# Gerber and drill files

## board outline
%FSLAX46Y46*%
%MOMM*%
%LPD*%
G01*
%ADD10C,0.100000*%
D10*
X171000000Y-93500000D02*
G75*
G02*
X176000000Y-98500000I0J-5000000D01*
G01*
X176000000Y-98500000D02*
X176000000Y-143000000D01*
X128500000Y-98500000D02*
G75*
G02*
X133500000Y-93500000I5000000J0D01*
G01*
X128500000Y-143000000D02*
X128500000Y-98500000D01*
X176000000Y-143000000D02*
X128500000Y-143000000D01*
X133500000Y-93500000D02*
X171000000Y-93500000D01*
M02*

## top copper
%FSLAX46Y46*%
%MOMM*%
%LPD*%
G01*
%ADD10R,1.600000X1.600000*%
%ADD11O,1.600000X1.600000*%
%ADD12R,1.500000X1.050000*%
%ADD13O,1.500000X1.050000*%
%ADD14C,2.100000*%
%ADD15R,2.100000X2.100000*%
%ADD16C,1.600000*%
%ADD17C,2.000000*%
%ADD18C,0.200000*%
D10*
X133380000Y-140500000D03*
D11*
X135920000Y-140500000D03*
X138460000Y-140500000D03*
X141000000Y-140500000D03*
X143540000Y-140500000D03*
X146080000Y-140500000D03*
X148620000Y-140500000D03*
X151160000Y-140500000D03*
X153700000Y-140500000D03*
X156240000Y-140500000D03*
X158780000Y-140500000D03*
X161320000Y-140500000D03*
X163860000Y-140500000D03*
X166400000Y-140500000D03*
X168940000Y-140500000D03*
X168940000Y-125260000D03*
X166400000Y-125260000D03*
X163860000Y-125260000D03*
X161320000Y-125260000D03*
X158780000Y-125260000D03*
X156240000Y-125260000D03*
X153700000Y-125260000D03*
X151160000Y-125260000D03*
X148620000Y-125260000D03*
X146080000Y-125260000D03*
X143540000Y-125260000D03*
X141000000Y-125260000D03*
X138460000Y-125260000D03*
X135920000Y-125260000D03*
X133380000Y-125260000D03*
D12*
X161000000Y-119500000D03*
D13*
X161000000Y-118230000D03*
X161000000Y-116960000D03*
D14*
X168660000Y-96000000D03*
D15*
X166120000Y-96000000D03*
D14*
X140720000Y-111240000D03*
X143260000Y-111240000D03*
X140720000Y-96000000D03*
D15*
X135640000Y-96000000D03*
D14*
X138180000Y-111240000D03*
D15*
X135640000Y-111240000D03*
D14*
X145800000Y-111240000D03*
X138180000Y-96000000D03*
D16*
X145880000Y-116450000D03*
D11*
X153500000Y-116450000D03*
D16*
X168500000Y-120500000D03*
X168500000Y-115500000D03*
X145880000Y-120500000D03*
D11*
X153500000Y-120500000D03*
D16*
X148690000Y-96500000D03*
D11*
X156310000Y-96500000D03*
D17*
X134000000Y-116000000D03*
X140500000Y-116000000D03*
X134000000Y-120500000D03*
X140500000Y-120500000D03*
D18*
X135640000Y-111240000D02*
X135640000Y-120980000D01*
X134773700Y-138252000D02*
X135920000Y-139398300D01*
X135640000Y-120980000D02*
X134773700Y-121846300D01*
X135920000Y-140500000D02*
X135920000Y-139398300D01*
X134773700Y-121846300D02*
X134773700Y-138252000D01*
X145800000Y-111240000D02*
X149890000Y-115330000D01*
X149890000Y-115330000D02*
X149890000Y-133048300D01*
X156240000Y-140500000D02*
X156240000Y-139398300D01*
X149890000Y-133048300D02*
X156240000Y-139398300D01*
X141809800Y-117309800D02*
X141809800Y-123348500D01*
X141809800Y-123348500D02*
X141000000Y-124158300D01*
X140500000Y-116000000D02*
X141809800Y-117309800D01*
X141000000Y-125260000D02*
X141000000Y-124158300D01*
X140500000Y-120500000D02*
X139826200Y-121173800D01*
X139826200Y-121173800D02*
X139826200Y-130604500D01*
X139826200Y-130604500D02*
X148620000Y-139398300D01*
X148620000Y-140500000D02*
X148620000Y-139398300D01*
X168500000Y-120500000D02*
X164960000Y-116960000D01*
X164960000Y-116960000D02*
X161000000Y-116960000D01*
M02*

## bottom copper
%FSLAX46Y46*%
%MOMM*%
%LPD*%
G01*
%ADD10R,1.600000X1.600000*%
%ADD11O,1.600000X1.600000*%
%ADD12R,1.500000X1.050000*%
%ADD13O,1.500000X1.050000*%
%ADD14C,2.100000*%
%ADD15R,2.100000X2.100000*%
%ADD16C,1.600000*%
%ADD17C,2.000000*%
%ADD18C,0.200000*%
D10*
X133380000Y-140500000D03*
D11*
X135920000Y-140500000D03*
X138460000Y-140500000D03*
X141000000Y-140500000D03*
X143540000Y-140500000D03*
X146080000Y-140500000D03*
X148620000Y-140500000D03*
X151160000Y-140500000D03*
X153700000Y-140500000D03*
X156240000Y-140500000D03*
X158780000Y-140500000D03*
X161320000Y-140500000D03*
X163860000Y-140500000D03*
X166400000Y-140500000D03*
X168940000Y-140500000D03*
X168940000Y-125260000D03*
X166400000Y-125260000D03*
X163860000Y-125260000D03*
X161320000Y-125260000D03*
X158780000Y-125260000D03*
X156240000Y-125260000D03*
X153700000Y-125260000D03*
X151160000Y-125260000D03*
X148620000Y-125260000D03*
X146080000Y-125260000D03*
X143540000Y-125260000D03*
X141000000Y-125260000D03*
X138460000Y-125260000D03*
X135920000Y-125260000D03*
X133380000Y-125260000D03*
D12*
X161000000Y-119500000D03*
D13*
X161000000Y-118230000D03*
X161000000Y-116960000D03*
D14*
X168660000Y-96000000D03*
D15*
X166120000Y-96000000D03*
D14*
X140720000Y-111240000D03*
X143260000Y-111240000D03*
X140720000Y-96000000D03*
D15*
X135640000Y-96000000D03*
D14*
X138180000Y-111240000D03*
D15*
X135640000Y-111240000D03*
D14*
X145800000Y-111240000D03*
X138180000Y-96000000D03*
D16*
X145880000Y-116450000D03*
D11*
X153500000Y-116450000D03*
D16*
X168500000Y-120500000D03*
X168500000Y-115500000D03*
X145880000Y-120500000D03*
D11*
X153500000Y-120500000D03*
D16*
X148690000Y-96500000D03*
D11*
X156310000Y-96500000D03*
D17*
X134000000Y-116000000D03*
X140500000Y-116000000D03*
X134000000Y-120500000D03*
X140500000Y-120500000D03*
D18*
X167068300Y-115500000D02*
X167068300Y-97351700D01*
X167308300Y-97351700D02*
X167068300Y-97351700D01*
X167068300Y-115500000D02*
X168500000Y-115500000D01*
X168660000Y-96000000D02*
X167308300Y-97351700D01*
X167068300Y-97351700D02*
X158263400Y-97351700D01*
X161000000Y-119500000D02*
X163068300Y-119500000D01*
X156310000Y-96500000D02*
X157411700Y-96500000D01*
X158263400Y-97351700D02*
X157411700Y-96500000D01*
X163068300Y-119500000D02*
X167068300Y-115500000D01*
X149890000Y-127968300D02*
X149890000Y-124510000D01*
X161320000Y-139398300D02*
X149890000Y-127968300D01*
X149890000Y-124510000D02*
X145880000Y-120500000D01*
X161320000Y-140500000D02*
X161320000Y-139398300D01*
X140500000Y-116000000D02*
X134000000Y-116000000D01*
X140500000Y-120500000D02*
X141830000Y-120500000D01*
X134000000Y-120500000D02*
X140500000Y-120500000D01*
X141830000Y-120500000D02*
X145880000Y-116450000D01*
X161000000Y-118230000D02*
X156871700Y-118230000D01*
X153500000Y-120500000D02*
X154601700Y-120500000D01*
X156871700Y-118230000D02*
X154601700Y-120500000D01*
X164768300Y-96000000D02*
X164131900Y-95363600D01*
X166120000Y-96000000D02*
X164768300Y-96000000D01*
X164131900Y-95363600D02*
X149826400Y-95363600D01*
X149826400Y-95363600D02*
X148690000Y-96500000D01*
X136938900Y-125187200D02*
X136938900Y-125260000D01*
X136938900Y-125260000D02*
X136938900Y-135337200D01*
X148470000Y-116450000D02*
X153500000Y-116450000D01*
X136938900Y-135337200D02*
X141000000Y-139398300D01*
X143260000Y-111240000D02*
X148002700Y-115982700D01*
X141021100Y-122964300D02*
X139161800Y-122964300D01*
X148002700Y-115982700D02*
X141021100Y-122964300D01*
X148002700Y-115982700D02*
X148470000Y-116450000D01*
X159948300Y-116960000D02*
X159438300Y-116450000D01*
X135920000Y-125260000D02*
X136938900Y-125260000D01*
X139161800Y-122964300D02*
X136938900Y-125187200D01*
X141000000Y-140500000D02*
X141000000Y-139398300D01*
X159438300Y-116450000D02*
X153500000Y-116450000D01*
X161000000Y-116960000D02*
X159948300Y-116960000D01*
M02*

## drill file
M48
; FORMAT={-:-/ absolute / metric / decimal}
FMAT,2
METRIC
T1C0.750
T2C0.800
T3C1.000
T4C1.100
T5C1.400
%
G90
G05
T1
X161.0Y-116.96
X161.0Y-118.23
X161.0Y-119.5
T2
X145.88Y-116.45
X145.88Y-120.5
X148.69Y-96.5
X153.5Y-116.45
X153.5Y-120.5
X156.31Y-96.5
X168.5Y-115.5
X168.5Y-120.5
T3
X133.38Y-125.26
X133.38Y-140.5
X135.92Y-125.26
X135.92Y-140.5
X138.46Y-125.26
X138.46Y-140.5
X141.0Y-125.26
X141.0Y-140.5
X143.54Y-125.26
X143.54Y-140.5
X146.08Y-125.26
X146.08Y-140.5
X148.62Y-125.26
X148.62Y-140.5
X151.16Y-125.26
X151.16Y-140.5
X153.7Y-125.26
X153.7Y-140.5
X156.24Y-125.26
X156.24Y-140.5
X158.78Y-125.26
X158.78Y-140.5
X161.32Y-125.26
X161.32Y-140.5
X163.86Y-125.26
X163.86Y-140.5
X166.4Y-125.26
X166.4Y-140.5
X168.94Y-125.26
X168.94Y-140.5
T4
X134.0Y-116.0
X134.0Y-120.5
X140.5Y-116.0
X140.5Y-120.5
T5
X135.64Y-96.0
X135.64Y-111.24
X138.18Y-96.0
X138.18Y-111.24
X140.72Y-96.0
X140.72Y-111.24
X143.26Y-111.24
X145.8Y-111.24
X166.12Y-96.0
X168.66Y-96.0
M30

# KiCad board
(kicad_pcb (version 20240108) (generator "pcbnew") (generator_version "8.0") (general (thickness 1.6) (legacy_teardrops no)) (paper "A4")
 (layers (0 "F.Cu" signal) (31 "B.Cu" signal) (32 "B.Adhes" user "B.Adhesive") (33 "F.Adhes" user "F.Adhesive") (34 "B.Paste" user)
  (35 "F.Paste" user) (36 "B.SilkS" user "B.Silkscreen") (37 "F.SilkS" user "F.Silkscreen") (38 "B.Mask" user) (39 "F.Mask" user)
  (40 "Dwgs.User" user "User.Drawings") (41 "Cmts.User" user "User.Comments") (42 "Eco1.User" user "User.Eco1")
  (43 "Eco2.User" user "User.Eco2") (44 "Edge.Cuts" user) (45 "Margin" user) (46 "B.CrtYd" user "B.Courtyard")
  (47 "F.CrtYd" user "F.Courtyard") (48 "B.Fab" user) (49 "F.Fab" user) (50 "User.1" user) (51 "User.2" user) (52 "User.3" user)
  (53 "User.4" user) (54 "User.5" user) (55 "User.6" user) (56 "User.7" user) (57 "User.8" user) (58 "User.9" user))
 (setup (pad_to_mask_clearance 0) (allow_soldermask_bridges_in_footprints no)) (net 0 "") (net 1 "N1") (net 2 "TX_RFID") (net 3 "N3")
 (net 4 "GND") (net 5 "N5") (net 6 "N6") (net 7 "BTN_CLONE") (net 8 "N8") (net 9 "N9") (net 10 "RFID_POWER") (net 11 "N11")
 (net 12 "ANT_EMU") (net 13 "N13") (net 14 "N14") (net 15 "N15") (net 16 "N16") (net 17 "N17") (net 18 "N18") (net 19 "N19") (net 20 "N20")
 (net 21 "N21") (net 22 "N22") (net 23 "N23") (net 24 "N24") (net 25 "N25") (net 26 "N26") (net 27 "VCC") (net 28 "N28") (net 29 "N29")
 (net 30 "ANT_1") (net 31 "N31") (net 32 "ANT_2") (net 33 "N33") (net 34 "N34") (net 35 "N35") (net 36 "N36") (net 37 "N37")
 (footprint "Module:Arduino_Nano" (layer "F.Cu") (at 133.38 140.5 90)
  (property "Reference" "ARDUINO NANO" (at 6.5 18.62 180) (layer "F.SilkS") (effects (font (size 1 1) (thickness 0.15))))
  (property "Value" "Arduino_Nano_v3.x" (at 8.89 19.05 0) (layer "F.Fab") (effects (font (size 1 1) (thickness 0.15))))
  (pad "1" thru_hole rect (at 0 0 90) (size 1.6 1.6) (drill 1) (layers "*.Cu" "*.Mask") (remove_unused_layers no) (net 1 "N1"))
  (pad "2" thru_hole oval (at 0 2.54 90) (size 1.6 1.6) (drill 1) (layers "*.Cu" "*.Mask") (remove_unused_layers no) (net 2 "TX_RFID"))
  (pad "3" thru_hole oval (at 0 5.08 90) (size 1.6 1.6) (drill 1) (layers "*.Cu" "*.Mask") (remove_unused_layers no) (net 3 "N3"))
  (pad "4" thru_hole oval (at 0 7.62 90) (size 1.6 1.6) (drill 1) (layers "*.Cu" "*.Mask") (remove_unused_layers no) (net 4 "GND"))
  (pad "5" thru_hole oval (at 0 10.16 90) (size 1.6 1.6) (drill 1) (layers "*.Cu" "*.Mask") (remove_unused_layers no) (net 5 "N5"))
  (pad "6" thru_hole oval (at 0 12.7 90) (size 1.6 1.6) (drill 1) (layers "*.Cu" "*.Mask") (remove_unused_layers no) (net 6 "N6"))
  (pad "7" thru_hole oval (at 0 15.24 90) (size 1.6 1.6) (drill 1) (layers "*.Cu" "*.Mask") (remove_unused_layers no) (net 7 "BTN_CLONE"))
  (pad "8" thru_hole oval (at 0 17.78 90) (size 1.6 1.6) (drill 1) (layers "*.Cu" "*.Mask") (remove_unused_layers no) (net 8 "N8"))
  (pad "9" thru_hole oval (at 0 20.32 90) (size 1.6 1.6) (drill 1) (layers "*.Cu" "*.Mask") (remove_unused_layers no) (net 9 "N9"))
  (pad "10" thru_hole oval (at 0 22.86 90) (size 1.6 1.6) (drill 1) (layers "*.Cu" "*.Mask") (remove_unused_layers no) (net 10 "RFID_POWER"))
  (pad "11" thru_hole oval (at 0 25.4 90) (size 1.6 1.6) (drill 1) (layers "*.Cu" "*.Mask") (remove_unused_layers no) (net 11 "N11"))
  (pad "12" thru_hole oval (at 0 27.94 90) (size 1.6 1.6) (drill 1) (layers "*.Cu" "*.Mask") (remove_unused_layers no) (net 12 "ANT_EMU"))
  (pad "13" thru_hole oval (at 0 30.48 90) (size 1.6 1.6) (drill 1) (layers "*.Cu" "*.Mask") (remove_unused_layers no) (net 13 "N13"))
  (pad "14" thru_hole oval (at 0 33.02 90) (size 1.6 1.6) (drill 1) (layers "*.Cu" "*.Mask") (remove_unused_layers no) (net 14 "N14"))
  (pad "15" thru_hole oval (at 0 35.56 90) (size 1.6 1.6) (drill 1) (layers "*.Cu" "*.Mask") (remove_unused_layers no) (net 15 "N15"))
  (pad "16" thru_hole oval (at 15.24 35.56 90) (size 1.6 1.6) (drill 1) (layers "*.Cu" "*.Mask") (remove_unused_layers no) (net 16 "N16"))
  (pad "17" thru_hole oval (at 15.24 33.02 90) (size 1.6 1.6) (drill 1) (layers "*.Cu" "*.Mask") (remove_unused_layers no) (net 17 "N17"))
  (pad "18" thru_hole oval (at 15.24 30.48 90) (size 1.6 1.6) (drill 1) (layers "*.Cu" "*.Mask") (remove_unused_layers no) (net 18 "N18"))
  (pad "19" thru_hole oval (at 15.24 27.94 90) (size 1.6 1.6) (drill 1) (layers "*.Cu" "*.Mask") (remove_unused_layers no) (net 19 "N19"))
  (pad "20" thru_hole oval (at 15.24 25.4 90) (size 1.6 1.6) (drill 1) (layers "*.Cu" "*.Mask") (remove_unused_layers no) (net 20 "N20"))
  (pad "21" thru_hole oval (at 15.24 22.86 90) (size 1.6 1.6) (drill 1) (layers "*.Cu" "*.Mask") (remove_unused_layers no) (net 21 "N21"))
  (pad "22" thru_hole oval (at 15.24 20.32 90) (size 1.6 1.6) (drill 1) (layers "*.Cu" "*.Mask") (remove_unused_layers no) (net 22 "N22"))
  (pad "23" thru_hole oval (at 15.24 17.78 90) (size 1.6 1.6) (drill 1) (layers "*.Cu" "*.Mask") (remove_unused_layers no) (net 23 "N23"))
  (pad "24" thru_hole oval (at 15.24 15.24 90) (size 1.6 1.6) (drill 1) (layers "*.Cu" "*.Mask") (remove_unused_layers no) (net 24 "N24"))
  (pad "25" thru_hole oval (at 15.24 12.7 90) (size 1.6 1.6) (drill 1) (layers "*.Cu" "*.Mask") (remove_unused_layers no) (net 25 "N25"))
  (pad "26" thru_hole oval (at 15.24 10.16 90) (size 1.6 1.6) (drill 1) (layers "*.Cu" "*.Mask") (remove_unused_layers no) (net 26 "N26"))
  (pad "27" thru_hole oval (at 15.24 7.62 90) (size 1.6 1.6) (drill 1) (layers "*.Cu" "*.Mask") (remove_unused_layers no) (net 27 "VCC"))
  (pad "28" thru_hole oval (at 15.24 5.08 90) (size 1.6 1.6) (drill 1) (layers "*.Cu" "*.Mask") (remove_unused_layers no) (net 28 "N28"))
  (pad "29" thru_hole oval (at 15.24 2.54 90) (size 1.6 1.6) (drill 1) (layers "*.Cu" "*.Mask") (remove_unused_layers no) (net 4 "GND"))
  (pad "30" thru_hole oval (at 15.24 0 90) (size 1.6 1.6) (drill 1) (layers "*.Cu" "*.Mask") (remove_unused_layers no) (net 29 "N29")))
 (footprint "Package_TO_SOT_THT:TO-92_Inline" (layer "F.Cu") (at 161 119.5 90)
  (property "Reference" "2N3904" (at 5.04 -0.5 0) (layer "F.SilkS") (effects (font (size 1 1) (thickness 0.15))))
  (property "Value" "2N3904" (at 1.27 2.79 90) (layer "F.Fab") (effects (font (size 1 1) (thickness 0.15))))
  (pad "1" thru_hole rect (at 0 0 90) (size 1.05 1.5) (drill 0.75) (layers "*.Cu" "*.Mask") (remove_unused_layers no) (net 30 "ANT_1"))
  (pad "2" thru_hole oval (at 1.27 0 90) (size 1.05 1.5) (drill 0.75) (layers "*.Cu" "*.Mask") (remove_unused_layers no) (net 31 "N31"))
  (pad "3" thru_hole oval (at 2.54 0 90) (size 1.05 1.5) (drill 0.75) (layers "*.Cu" "*.Mask") (remove_unused_layers no) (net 4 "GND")))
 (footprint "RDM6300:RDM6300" (layer "F.Cu") (at 152.15 103.62 180)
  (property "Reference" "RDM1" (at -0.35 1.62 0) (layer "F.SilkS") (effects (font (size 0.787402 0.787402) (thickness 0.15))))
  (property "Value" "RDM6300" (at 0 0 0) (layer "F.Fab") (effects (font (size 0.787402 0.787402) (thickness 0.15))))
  (pad "ANT1" thru_hole circle (at -16.51 7.62 180) (size 2.1 2.1) (drill 1.4) (layers "*.Cu" "*.Mask") (remove_unused_layers no)
   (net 30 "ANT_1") (solder_mask_margin 0.102))
  (pad "ANT2" thru_hole rect (at -13.97 7.62 180) (size 2.1 2.1) (drill 1.4) (layers "*.Cu" "*.Mask") (remove_unused_layers no)
   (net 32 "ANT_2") (solder_mask_margin 0.102))
  (pad "D0" thru_hole circle (at 11.43 -7.62 180) (size 2.1 2.1) (drill 1.4) (layers "*.Cu" "*.Mask") (remove_unused_layers no)
   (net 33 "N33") (solder_mask_margin 0.102))
  (pad "GND" thru_hole circle (at 8.89 -7.62 180) (size 2.1 2.1) (drill 1.4) (layers "*.Cu" "*.Mask") (remove_unused_layers no)
   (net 4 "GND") (solder_mask_margin 0.102))
  (pad "GND1" thru_hole circle (at 11.43 7.62 180) (size 2.1 2.1) (drill 1.4) (layers "*.Cu" "*.Mask") (remove_unused_layers no)
   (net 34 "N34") (solder_mask_margin 0.102))
  (pad "LED" thru_hole rect (at 16.51 7.62 180) (size 2.1 2.1) (drill 1.4) (layers "*.Cu" "*.Mask") (remove_unused_layers no) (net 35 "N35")
   (solder_mask_margin 0.102))
  (pad "RX" thru_hole circle (at 13.97 -7.62 180) (size 2.1 2.1) (drill 1.4) (layers "*.Cu" "*.Mask") (remove_unused_layers no)
   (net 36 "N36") (solder_mask_margin 0.102))
  (pad "TX" thru_hole rect (at 16.51 -7.62 180) (size 2.1 2.1) (drill 1.4) (layers "*.Cu" "*.Mask") (remove_unused_layers no)
   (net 2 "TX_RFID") (solder_mask_margin 0.102))
  (pad "VCC" thru_hole circle (at 6.35 -7.62 180) (size 2.1 2.1) (drill 1.4) (layers "*.Cu" "*.Mask") (remove_unused_layers no)
   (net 10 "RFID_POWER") (solder_mask_margin 0.102))
  (pad "VCC1" thru_hole circle (at 13.97 7.62 180) (size 2.1 2.1) (drill 1.4) (layers "*.Cu" "*.Mask") (remove_unused_layers no)
   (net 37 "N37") (solder_mask_margin 0.102)))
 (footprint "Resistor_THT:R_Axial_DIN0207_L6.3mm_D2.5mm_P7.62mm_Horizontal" (layer "F.Cu") (at 145.88 116.45)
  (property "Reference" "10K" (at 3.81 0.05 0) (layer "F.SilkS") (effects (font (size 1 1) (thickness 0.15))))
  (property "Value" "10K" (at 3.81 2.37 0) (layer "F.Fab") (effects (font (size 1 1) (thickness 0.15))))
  (pad "1" thru_hole circle (at 0 0) (size 1.6 1.6) (drill 0.8) (layers "*.Cu" "*.Mask") (remove_unused_layers no) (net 7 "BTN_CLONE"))
  (pad "2" thru_hole oval (at 7.62 0) (size 1.6 1.6) (drill 0.8) (layers "*.Cu" "*.Mask") (remove_unused_layers no) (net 4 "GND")))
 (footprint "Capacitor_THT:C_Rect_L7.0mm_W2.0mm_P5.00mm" (layer "F.Cu") (at 168.5 120.5 90)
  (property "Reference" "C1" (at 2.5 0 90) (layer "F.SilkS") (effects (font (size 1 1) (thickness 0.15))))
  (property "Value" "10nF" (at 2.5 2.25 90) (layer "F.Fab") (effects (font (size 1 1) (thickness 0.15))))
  (pad "1" thru_hole circle (at 0 0 90) (size 1.6 1.6) (drill 0.8) (layers "*.Cu" "*.Mask") (remove_unused_layers no) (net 4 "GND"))
  (pad "2" thru_hole circle (at 5 0 90) (size 1.6 1.6) (drill 0.8) (layers "*.Cu" "*.Mask") (remove_unused_layers no) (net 30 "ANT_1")))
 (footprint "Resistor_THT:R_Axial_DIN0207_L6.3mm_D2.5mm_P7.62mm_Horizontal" (layer "F.Cu") (at 145.88 120.5)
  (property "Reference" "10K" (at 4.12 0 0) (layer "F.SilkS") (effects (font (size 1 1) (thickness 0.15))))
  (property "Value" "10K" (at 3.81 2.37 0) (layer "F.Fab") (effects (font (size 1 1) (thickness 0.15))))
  (pad "1" thru_hole circle (at 0 0) (size 1.6 1.6) (drill 0.8) (layers "*.Cu" "*.Mask") (remove_unused_layers no) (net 12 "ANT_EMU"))
  (pad "2" thru_hole oval (at 7.62 0) (size 1.6 1.6) (drill 0.8) (layers "*.Cu" "*.Mask") (remove_unused_layers no) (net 31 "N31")))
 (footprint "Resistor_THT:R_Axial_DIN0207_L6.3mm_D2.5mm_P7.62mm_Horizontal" (layer "F.Cu") (at 148.69 96.5)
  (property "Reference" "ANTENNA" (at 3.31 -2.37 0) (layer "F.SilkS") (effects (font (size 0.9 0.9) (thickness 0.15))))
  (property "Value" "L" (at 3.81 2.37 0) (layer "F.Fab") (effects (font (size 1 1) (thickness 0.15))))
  (pad "1" thru_hole circle (at 0 0) (size 1.6 1.6) (drill 0.8) (layers "*.Cu" "*.Mask") (remove_unused_layers no) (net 32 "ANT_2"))
  (pad "2" thru_hole oval (at 7.62 0) (size 1.6 1.6) (drill 0.8) (layers "*.Cu" "*.Mask") (remove_unused_layers no) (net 30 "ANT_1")))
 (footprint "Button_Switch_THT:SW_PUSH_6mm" (layer "F.Cu") (at 134 116)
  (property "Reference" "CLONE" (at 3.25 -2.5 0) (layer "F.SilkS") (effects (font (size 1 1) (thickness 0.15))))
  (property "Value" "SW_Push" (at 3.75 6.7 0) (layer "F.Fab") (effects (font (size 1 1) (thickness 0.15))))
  (pad "1" thru_hole circle (at 0 0 90) (size 2 2) (drill 1.1) (layers "*.Cu" "*.Mask") (remove_unused_layers no) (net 27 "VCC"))
  (pad "1" thru_hole circle (at 6.5 0 90) (size 2 2) (drill 1.1) (layers "*.Cu" "*.Mask") (remove_unused_layers no) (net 27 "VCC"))
  (pad "2" thru_hole circle (at 0 4.5 90) (size 2 2) (drill 1.1) (layers "*.Cu" "*.Mask") (remove_unused_layers no) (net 7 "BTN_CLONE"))
  (pad "2" thru_hole circle (at 6.5 4.5 90) (size 2 2) (drill 1.1) (layers "*.Cu" "*.Mask") (remove_unused_layers no) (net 7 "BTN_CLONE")))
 (gr_arc (start 171 93.5) (mid 174.535534 94.964466) (end 176 98.5) (stroke (width 0.1) (type default)) (layer "Edge.Cuts"))
 (gr_line (start 176 98.5) (end 176 143) (stroke (width 0.1) (type default)) (layer "Edge.Cuts"))
 (gr_arc (start 128.5 98.5) (mid 129.964466 94.964466) (end 133.5 93.5) (stroke (width 0.1) (type default)) (layer "Edge.Cuts"))
 (gr_line (start 128.5 143) (end 128.5 98.5) (stroke (width 0.1) (type default)) (layer "Edge.Cuts"))
 (gr_line (start 176 143) (end 128.5 143) (stroke (width 0.1) (type default)) (layer "Edge.Cuts"))
 (gr_line (start 133.5 93.5) (end 171 93.5) (stroke (width 0.1) (type default)) (layer "Edge.Cuts"))
 (segment (start 167.0683 115.5) (end 167.0683 97.3517) (width 0.2) (layer "B.Cu") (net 30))
 (segment (start 167.3083 97.3517) (end 167.0683 97.3517) (width 0.2) (layer "B.Cu") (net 30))
 (segment (start 167.0683 115.5) (end 168.5 115.5) (width 0.2) (layer "B.Cu") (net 30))
 (segment (start 168.66 96) (end 167.3083 97.3517) (width 0.2) (layer "B.Cu") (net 30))
 (segment (start 167.0683 97.3517) (end 158.2634 97.3517) (width 0.2) (layer "B.Cu") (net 30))
 (segment (start 161 119.5) (end 163.0683 119.5) (width 0.2) (layer "B.Cu") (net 30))
 (segment (start 156.31 96.5) (end 157.4117 96.5) (width 0.2) (layer "B.Cu") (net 30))
 (segment (start 158.2634 97.3517) (end 157.4117 96.5) (width 0.2) (layer "B.Cu") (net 30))
 (segment (start 163.0683 119.5) (end 167.0683 115.5) (width 0.2) (layer "B.Cu") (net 30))
 (segment (start 149.89 127.9683) (end 149.89 124.51) (width 0.2) (layer "B.Cu") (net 12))
 (segment (start 161.32 139.3983) (end 149.89 127.9683) (width 0.2) (layer "B.Cu") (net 12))
 (segment (start 149.89 124.51) (end 145.88 120.5) (width 0.2) (layer "B.Cu") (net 12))
 (segment (start 161.32 140.5) (end 161.32 139.3983) (width 0.2) (layer "B.Cu") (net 12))
 (segment (start 135.64 111.24) (end 135.64 120.98) (width 0.2) (layer "F.Cu") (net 2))
 (segment (start 134.7737 138.252) (end 135.92 139.3983) (width 0.2) (layer "F.Cu") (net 2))
 (segment (start 135.64 120.98) (end 134.7737 121.8463) (width 0.2) (layer "F.Cu") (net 2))
 (segment (start 135.92 140.5) (end 135.92 139.3983) (width 0.2) (layer "F.Cu") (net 2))
 (segment (start 134.7737 121.8463) (end 134.7737 138.252) (width 0.2) (layer "F.Cu") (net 2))
 (segment (start 145.8 111.24) (end 149.89 115.33) (width 0.2) (layer "F.Cu") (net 10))
 (segment (start 149.89 115.33) (end 149.89 133.0483) (width 0.2) (layer "F.Cu") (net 10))
 (segment (start 156.24 140.5) (end 156.24 139.3983) (width 0.2) (layer "F.Cu") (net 10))
 (segment (start 149.89 133.0483) (end 156.24 139.3983) (width 0.2) (layer "F.Cu") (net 10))
 (segment (start 141.8098 117.3098) (end 141.8098 123.3485) (width 0.2) (layer "F.Cu") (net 27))
 (segment (start 141.8098 123.3485) (end 141 124.1583) (width 0.2) (layer "F.Cu") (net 27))
 (segment (start 140.5 116) (end 141.8098 117.3098) (width 0.2) (layer "F.Cu") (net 27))
 (segment (start 141 125.26) (end 141 124.1583) (width 0.2) (layer "F.Cu") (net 27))
 (segment (start 140.5 116) (end 134 116) (width 0.2) (layer "B.Cu") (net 27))
 (segment (start 140.5 120.5) (end 139.8262 121.1738) (width 0.2) (layer "F.Cu") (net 7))
 (segment (start 139.8262 121.1738) (end 139.8262 130.6045) (width 0.2) (layer "F.Cu") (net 7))
 (segment (start 139.8262 130.6045) (end 148.62 139.3983) (width 0.2) (layer "F.Cu") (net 7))
 (segment (start 148.62 140.5) (end 148.62 139.3983) (width 0.2) (layer "F.Cu") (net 7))
 (segment (start 140.5 120.5) (end 141.83 120.5) (width 0.2) (layer "B.Cu") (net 7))
 (segment (start 134 120.5) (end 140.5 120.5) (width 0.2) (layer "B.Cu") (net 7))
 (segment (start 141.83 120.5) (end 145.88 116.45) (width 0.2) (layer "B.Cu") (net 7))
 (segment (start 161 118.23) (end 156.8717 118.23) (width 0.2) (layer "B.Cu") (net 31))
 (segment (start 153.5 120.5) (end 154.6017 120.5) (width 0.2) (layer "B.Cu") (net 31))
 (segment (start 156.8717 118.23) (end 154.6017 120.5) (width 0.2) (layer "B.Cu") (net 31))
 (segment (start 164.7683 96) (end 164.1319 95.3636) (width 0.2) (layer "B.Cu") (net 32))
 (segment (start 166.12 96) (end 164.7683 96) (width 0.2) (layer "B.Cu") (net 32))
 (segment (start 164.1319 95.3636) (end 149.8264 95.3636) (width 0.2) (layer "B.Cu") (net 32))
 (segment (start 149.8264 95.3636) (end 148.69 96.5) (width 0.2) (layer "B.Cu") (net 32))
 (segment (start 168.5 120.5) (end 164.96 116.96) (width 0.2) (layer "F.Cu") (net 4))
 (segment (start 164.96 116.96) (end 161 116.96) (width 0.2) (layer "F.Cu") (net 4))
 (segment (start 136.9389 125.1872) (end 136.9389 125.26) (width 0.2) (layer "B.Cu") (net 4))
 (segment (start 136.9389 125.26) (end 136.9389 135.3372) (width 0.2) (layer "B.Cu") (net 4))
 (segment (start 148.47 116.45) (end 153.5 116.45) (width 0.2) (layer "B.Cu") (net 4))
 (segment (start 136.9389 135.3372) (end 141 139.3983) (width 0.2) (layer "B.Cu") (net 4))
 (segment (start 143.26 111.24) (end 148.0027 115.9827) (width 0.2) (layer "B.Cu") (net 4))
 (segment (start 141.0211 122.9643) (end 139.1618 122.9643) (width 0.2) (layer "B.Cu") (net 4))
 (segment (start 148.0027 115.9827) (end 141.0211 122.9643) (width 0.2) (layer "B.Cu") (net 4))
 (segment (start 148.0027 115.9827) (end 148.47 116.45) (width 0.2) (layer "B.Cu") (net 4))
 (segment (start 159.9483 116.96) (end 159.4383 116.45) (width 0.2) (layer "B.Cu") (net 4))
 (segment (start 135.92 125.26) (end 136.9389 125.26) (width 0.2) (layer "B.Cu") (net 4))
 (segment (start 139.1618 122.9643) (end 136.9389 125.1872) (width 0.2) (layer "B.Cu") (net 4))
 (segment (start 141 140.5) (end 141 139.3983) (width 0.2) (layer "B.Cu") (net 4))
 (segment (start 159.4383 116.45) (end 153.5 116.45) (width 0.2) (layer "B.Cu") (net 4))
 (segment (start 161 116.96) (end 159.9483 116.96) (width 0.2) (layer "B.Cu") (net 4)))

